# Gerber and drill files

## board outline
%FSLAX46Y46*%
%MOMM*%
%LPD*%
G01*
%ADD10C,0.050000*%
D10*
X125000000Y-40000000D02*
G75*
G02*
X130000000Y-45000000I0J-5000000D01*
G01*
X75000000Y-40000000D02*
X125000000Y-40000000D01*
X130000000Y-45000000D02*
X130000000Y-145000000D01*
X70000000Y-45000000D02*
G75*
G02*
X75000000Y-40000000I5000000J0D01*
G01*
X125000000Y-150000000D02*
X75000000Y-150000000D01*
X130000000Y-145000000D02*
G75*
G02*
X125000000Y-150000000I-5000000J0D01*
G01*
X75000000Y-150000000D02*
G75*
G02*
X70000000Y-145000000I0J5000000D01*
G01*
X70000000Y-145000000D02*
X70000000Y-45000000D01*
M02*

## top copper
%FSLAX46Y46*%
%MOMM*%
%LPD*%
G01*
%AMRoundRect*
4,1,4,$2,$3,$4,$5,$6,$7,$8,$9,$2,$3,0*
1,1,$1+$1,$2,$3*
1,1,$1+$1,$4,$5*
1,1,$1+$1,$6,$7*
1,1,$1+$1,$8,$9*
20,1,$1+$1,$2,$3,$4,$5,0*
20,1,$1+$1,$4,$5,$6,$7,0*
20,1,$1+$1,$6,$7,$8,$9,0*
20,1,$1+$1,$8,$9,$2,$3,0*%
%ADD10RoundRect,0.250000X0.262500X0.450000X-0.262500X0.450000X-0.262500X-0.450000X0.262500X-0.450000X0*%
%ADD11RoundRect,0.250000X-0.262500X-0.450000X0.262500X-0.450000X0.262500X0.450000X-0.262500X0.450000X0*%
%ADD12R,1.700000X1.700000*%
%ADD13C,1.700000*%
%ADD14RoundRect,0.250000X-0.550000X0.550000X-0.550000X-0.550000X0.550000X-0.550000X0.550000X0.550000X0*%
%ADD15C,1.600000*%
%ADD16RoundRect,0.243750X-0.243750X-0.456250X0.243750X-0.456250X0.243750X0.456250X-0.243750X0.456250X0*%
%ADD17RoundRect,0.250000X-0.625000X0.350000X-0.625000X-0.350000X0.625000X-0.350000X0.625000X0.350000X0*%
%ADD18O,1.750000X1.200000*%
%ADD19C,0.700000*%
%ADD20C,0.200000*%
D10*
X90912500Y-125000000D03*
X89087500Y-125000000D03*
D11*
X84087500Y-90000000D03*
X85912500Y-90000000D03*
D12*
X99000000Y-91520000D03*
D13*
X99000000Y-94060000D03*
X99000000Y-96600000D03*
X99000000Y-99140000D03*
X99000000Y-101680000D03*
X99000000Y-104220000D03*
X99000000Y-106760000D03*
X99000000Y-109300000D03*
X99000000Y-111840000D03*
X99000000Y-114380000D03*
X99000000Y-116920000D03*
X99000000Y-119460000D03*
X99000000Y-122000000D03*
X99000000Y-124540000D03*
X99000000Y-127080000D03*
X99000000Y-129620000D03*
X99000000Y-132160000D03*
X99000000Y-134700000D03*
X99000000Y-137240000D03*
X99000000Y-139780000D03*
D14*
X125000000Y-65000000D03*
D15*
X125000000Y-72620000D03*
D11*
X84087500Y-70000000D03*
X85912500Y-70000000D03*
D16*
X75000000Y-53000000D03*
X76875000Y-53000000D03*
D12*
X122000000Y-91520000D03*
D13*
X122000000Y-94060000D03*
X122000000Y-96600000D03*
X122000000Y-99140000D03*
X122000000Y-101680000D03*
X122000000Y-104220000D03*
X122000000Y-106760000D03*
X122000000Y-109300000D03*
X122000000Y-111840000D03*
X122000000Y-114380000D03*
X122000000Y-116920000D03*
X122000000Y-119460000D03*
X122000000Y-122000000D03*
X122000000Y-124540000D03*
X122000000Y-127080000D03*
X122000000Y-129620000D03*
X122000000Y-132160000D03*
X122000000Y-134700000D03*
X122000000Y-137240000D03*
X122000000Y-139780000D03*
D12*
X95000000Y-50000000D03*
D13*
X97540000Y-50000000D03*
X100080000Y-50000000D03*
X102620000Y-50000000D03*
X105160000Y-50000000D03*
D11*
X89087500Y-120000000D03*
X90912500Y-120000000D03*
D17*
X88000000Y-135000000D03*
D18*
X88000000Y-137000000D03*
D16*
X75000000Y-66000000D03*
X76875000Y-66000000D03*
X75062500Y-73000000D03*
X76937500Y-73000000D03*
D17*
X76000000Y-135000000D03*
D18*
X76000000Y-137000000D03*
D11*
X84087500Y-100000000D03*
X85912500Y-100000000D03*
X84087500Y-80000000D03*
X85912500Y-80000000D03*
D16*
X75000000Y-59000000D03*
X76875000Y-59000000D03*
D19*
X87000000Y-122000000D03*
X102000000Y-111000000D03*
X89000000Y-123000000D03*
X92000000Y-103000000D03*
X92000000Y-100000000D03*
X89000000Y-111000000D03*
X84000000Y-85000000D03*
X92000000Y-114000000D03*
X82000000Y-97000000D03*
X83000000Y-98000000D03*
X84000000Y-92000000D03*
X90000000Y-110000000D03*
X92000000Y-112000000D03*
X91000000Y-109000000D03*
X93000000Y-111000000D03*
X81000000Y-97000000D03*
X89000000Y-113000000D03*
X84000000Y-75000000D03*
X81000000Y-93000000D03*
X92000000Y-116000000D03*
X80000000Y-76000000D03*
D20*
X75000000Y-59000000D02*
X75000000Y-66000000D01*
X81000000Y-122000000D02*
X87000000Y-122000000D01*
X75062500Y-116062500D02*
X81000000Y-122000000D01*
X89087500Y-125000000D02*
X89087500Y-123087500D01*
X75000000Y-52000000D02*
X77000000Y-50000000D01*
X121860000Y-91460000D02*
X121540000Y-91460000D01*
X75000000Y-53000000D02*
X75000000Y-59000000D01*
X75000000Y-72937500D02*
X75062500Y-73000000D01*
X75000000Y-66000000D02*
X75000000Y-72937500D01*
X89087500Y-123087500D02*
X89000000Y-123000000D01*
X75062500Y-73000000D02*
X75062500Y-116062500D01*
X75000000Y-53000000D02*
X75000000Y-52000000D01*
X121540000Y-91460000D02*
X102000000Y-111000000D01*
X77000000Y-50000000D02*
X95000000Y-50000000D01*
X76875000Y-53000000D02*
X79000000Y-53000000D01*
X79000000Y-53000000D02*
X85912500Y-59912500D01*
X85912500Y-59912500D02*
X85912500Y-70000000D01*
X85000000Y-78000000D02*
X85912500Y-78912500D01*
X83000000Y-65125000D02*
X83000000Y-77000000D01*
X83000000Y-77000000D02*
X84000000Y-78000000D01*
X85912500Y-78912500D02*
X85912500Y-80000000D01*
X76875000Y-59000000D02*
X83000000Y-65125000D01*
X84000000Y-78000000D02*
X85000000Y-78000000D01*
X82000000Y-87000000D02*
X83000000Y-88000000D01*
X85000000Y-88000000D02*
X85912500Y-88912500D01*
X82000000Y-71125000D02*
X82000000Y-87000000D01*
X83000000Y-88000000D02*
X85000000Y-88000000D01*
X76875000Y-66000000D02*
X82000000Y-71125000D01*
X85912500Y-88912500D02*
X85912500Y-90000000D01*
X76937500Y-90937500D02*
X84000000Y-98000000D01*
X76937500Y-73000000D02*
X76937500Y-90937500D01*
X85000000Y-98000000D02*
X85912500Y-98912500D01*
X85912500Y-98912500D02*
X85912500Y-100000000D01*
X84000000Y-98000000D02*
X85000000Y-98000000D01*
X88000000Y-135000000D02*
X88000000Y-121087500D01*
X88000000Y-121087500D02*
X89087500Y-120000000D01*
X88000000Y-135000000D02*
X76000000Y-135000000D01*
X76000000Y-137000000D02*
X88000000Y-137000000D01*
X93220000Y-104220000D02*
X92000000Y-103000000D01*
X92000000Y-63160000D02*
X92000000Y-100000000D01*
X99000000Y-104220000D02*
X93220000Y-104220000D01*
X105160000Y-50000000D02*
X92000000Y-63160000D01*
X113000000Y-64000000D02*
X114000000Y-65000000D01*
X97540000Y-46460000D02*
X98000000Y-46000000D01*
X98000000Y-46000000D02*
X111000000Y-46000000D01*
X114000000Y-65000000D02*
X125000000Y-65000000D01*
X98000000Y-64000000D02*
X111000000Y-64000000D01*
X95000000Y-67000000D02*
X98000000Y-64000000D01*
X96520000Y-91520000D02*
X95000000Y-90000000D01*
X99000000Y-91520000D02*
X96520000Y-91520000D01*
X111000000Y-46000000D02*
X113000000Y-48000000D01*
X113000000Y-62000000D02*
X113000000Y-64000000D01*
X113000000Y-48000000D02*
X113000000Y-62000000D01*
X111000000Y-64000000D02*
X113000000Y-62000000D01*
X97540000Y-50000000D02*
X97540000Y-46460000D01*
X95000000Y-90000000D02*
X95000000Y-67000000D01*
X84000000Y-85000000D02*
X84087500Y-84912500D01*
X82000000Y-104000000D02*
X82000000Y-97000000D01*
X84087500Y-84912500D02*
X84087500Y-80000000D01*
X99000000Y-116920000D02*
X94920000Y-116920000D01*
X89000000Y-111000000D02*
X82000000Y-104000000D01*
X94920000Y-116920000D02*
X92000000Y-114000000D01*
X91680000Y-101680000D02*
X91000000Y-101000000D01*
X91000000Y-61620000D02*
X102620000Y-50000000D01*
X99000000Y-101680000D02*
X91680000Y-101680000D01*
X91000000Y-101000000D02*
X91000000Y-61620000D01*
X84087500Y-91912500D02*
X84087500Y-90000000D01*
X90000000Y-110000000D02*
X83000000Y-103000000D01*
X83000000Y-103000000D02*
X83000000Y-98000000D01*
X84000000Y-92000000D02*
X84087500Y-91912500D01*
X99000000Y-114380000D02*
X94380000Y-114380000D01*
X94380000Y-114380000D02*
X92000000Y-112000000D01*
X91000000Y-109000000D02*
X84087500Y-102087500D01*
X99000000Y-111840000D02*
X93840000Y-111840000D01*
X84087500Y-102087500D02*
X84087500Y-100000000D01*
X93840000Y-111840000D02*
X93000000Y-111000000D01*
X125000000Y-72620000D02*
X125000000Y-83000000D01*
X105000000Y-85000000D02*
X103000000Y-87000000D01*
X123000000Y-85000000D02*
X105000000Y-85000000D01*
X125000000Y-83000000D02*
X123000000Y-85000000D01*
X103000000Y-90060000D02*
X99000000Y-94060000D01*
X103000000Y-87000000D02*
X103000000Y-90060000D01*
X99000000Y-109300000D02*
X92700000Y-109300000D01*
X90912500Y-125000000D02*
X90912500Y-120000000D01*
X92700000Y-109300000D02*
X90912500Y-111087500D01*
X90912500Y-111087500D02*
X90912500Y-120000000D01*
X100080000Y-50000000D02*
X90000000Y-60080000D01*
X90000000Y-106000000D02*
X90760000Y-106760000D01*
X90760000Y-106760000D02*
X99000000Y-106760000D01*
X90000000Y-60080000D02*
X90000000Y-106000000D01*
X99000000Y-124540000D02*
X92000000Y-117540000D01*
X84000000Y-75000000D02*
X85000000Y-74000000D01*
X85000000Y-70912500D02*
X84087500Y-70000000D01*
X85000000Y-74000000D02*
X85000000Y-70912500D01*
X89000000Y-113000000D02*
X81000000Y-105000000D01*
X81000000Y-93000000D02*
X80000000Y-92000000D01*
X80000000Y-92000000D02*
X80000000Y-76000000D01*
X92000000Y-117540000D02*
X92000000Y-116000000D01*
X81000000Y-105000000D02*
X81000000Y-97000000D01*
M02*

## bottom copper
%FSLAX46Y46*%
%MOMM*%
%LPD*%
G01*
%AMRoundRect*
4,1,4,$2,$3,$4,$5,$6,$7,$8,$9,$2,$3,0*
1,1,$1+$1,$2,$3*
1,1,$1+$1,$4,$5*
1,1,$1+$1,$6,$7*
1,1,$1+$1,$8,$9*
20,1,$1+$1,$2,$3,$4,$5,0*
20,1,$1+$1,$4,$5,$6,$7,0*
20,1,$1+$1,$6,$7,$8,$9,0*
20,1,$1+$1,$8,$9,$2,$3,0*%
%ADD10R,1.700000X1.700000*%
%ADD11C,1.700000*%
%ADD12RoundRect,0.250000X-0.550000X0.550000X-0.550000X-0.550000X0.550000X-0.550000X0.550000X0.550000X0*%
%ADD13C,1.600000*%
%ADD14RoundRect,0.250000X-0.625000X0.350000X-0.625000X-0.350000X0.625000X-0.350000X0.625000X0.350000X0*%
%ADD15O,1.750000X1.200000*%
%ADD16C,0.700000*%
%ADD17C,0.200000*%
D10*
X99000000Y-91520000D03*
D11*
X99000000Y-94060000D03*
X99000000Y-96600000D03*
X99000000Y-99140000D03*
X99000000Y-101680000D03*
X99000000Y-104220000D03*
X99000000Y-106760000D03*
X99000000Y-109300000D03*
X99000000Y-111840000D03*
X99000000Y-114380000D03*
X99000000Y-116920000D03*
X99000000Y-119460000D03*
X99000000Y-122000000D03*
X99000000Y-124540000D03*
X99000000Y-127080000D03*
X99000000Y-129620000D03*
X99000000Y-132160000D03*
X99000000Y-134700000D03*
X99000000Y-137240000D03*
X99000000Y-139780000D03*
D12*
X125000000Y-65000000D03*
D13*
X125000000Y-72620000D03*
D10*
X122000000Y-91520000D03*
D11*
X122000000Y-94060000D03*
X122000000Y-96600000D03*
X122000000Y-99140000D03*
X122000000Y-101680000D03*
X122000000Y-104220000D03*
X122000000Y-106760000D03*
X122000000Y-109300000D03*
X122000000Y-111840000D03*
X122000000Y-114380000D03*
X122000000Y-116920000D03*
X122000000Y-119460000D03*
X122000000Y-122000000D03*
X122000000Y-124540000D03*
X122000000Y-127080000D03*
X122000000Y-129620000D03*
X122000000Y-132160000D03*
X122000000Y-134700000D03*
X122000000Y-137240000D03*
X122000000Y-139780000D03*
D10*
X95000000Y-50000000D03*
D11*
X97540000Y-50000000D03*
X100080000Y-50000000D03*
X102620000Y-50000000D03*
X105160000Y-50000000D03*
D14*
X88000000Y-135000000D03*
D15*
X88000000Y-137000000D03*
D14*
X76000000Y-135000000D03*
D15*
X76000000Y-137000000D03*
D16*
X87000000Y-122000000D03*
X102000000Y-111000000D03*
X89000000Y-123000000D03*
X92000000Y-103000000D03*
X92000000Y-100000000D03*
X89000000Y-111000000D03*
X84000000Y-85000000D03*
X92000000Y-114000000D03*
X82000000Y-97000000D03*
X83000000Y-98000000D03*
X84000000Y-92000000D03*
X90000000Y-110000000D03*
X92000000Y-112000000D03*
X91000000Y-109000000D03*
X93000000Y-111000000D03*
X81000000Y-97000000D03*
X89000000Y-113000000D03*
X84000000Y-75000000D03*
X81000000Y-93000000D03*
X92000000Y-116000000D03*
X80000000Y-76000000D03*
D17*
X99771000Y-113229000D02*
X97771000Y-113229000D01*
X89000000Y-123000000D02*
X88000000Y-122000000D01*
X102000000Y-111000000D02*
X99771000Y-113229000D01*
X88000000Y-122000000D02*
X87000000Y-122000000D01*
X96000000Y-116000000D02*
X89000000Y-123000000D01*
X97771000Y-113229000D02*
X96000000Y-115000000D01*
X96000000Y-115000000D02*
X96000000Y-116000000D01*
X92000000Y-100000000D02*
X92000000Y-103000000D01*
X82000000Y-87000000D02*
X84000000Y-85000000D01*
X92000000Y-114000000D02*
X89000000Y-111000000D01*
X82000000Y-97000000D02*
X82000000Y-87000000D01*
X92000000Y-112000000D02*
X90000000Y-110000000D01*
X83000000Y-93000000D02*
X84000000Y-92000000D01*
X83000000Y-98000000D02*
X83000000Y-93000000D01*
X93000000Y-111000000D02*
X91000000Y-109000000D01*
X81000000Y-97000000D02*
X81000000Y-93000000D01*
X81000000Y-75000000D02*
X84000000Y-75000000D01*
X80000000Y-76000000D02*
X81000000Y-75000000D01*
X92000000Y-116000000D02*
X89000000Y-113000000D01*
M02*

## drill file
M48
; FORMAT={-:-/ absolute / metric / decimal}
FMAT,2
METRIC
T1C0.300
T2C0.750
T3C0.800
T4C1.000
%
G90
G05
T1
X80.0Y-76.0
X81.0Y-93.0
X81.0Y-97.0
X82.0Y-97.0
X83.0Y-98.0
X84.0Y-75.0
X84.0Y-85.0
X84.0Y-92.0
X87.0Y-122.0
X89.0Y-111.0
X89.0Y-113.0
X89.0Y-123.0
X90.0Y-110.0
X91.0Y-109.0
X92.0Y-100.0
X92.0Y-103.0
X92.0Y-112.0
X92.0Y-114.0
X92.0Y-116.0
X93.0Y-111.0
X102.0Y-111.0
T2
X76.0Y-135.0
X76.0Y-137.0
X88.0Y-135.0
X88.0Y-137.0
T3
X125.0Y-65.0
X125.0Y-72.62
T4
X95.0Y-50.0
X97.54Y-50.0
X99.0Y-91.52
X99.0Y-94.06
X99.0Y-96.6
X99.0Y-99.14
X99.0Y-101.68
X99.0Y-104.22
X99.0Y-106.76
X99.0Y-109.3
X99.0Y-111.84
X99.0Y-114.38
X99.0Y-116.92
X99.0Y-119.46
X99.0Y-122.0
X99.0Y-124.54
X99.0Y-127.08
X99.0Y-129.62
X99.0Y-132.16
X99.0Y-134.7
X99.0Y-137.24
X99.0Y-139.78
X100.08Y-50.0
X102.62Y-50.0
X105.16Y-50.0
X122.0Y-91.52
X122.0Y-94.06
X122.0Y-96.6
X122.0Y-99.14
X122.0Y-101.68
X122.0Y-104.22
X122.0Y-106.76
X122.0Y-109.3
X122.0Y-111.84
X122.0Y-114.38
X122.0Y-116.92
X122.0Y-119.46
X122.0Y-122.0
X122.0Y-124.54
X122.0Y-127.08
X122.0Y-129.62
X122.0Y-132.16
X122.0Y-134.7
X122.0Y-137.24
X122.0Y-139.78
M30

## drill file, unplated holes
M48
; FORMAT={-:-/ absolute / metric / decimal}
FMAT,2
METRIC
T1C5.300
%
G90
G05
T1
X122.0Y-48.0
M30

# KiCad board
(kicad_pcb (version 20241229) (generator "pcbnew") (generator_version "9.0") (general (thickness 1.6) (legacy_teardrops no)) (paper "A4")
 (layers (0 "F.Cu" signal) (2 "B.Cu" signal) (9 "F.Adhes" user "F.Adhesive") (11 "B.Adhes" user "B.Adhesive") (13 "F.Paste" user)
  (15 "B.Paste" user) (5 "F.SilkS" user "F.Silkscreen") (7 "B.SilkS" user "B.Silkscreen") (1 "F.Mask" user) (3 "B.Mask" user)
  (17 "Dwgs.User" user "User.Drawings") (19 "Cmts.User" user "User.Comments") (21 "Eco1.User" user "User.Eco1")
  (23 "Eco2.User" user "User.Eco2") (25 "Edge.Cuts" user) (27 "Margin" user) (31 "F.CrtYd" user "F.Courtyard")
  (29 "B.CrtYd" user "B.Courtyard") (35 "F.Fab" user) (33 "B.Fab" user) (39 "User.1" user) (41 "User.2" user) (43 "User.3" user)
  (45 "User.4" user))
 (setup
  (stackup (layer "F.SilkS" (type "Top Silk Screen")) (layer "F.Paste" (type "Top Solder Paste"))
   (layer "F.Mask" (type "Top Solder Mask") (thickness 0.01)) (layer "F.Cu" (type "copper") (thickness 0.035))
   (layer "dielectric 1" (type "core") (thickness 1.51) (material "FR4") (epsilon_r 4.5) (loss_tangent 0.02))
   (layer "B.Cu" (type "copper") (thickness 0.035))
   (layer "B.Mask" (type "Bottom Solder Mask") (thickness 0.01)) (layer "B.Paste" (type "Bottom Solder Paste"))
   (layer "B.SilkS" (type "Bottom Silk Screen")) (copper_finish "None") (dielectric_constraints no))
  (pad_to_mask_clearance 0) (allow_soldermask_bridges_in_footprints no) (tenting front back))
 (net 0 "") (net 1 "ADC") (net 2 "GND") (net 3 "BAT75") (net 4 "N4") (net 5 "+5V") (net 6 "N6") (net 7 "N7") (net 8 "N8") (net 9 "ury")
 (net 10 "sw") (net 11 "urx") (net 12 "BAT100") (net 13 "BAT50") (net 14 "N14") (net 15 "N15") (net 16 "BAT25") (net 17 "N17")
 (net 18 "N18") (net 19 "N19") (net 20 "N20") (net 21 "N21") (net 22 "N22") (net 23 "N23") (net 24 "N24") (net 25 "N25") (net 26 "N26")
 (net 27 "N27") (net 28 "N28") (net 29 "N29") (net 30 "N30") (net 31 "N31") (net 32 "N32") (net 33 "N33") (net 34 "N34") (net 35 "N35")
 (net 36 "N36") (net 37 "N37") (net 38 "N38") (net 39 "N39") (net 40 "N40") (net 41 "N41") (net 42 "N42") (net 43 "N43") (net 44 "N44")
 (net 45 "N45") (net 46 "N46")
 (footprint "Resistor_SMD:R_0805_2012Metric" (layer "F.Cu") (at 90 125 180)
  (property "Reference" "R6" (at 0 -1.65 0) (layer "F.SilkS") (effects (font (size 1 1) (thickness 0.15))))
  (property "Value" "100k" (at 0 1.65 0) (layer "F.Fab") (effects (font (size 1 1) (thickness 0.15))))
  (pad "1" smd roundrect (at -0.9125 0 180) (size 1.025 1.4) (layers "F.Cu" "F.Mask" "F.Paste") (roundrect_rratio 0.243902) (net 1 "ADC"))
  (pad "2" smd roundrect (at 0.9125 0 180) (size 1.025 1.4) (layers "F.Cu" "F.Mask" "F.Paste") (roundrect_rratio 0.243902) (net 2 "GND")))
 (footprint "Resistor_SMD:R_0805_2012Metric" (layer "F.Cu") (at 85 90)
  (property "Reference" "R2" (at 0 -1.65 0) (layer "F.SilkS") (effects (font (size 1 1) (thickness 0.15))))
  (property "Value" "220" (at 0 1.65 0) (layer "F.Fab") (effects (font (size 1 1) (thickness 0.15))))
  (pad "1" smd roundrect (at -0.9125 0) (size 1.025 1.4) (layers "F.Cu" "F.Mask" "F.Paste") (roundrect_rratio 0.243902) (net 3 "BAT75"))
  (pad "2" smd roundrect (at 0.9125 0) (size 1.025 1.4) (layers "F.Cu" "F.Mask" "F.Paste") (roundrect_rratio 0.243902) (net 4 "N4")))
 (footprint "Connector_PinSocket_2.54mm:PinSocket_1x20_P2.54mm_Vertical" (layer "F.Cu") (at 99 91.52)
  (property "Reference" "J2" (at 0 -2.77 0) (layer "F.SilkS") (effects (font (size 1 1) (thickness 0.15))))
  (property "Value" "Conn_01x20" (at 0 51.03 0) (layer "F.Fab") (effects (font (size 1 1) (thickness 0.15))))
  (pad "1" thru_hole rect (at 0 0) (size 1.7 1.7) (drill 1) (layers "*.Cu" "*.Mask") (remove_unused_layers no) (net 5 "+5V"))
  (pad "2" thru_hole circle (at 0 2.54) (size 1.7 1.7) (drill 1) (layers "*.Cu" "*.Mask") (remove_unused_layers no) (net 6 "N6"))
  (pad "3" thru_hole circle (at 0 5.08) (size 1.7 1.7) (drill 1) (layers "*.Cu" "*.Mask") (remove_unused_layers no) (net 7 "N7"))
  (pad "4" thru_hole circle (at 0 7.62) (size 1.7 1.7) (drill 1) (layers "*.Cu" "*.Mask") (remove_unused_layers no) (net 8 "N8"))
  (pad "5" thru_hole circle (at 0 10.16) (size 1.7 1.7) (drill 1) (layers "*.Cu" "*.Mask") (remove_unused_layers no) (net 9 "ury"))
  (pad "6" thru_hole circle (at 0 12.7) (size 1.7 1.7) (drill 1) (layers "*.Cu" "*.Mask") (remove_unused_layers no) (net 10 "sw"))
  (pad "7" thru_hole circle (at 0 15.24) (size 1.7 1.7) (drill 1) (layers "*.Cu" "*.Mask") (remove_unused_layers no) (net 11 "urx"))
  (pad "8" thru_hole circle (at 0 17.78) (size 1.7 1.7) (drill 1) (layers "*.Cu" "*.Mask") (remove_unused_layers no) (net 1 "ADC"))
  (pad "9" thru_hole circle (at 0 20.32) (size 1.7 1.7) (drill 1) (layers "*.Cu" "*.Mask") (remove_unused_layers no) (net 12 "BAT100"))
  (pad "10" thru_hole circle (at 0 22.86) (size 1.7 1.7) (drill 1) (layers "*.Cu" "*.Mask") (remove_unused_layers no) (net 3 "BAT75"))
  (pad "11" thru_hole circle (at 0 25.4) (size 1.7 1.7) (drill 1) (layers "*.Cu" "*.Mask") (remove_unused_layers no) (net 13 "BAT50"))
  (pad "12" thru_hole circle (at 0 27.94) (size 1.7 1.7) (drill 1) (layers "*.Cu" "*.Mask") (remove_unused_layers no) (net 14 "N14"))
  (pad "13" thru_hole circle (at 0 30.48) (size 1.7 1.7) (drill 1) (layers "*.Cu" "*.Mask") (remove_unused_layers no) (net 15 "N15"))
  (pad "14" thru_hole circle (at 0 33.02) (size 1.7 1.7) (drill 1) (layers "*.Cu" "*.Mask") (remove_unused_layers no) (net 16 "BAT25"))
  (pad "15" thru_hole circle (at 0 35.56) (size 1.7 1.7) (drill 1) (layers "*.Cu" "*.Mask") (remove_unused_layers no) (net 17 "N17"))
  (pad "16" thru_hole circle (at 0 38.1) (size 1.7 1.7) (drill 1) (layers "*.Cu" "*.Mask") (remove_unused_layers no) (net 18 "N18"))
  (pad "17" thru_hole circle (at 0 40.64) (size 1.7 1.7) (drill 1) (layers "*.Cu" "*.Mask") (remove_unused_layers no) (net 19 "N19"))
  (pad "18" thru_hole circle (at 0 43.18) (size 1.7 1.7) (drill 1) (layers "*.Cu" "*.Mask") (remove_unused_layers no) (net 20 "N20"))
  (pad "19" thru_hole circle (at 0 45.72) (size 1.7 1.7) (drill 1) (layers "*.Cu" "*.Mask") (remove_unused_layers no) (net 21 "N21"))
  (pad "20" thru_hole circle (at 0 48.26) (size 1.7 1.7) (drill 1) (layers "*.Cu" "*.Mask") (remove_unused_layers no) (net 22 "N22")))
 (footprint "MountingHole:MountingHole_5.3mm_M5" (layer "F.Cu") (at 122 48)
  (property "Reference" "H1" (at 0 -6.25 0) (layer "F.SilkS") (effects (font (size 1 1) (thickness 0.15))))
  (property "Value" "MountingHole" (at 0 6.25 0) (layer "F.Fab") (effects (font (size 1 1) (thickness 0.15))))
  (pad "" np_thru_hole circle (at 0 0) (size 5.3 5.3) (drill 5.3) (layers "*.Cu" "*.Mask")))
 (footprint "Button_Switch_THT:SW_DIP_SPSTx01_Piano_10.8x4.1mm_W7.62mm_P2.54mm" (layer "F.Cu") (at 125 65 -90)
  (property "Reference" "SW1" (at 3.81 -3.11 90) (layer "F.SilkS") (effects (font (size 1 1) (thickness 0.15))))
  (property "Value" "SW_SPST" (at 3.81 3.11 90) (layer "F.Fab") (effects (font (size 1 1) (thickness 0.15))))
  (pad "1" thru_hole roundrect (at 0 0 270) (size 1.6 1.6) (drill 0.8) (layers "*.Cu" "*.Mask") (remove_unused_layers no)
   (roundrect_rratio 0.15625) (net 5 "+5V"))
  (pad "2" thru_hole circle (at 7.62 0 270) (size 1.6 1.6) (drill 0.8) (layers "*.Cu" "*.Mask") (remove_unused_layers no) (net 6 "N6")))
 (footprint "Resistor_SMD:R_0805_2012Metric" (layer "F.Cu") (at 85 70)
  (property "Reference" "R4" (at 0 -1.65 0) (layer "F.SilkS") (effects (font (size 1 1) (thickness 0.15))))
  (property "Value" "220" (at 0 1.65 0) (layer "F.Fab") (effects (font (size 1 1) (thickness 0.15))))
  (pad "1" smd roundrect (at -0.9125 0) (size 1.025 1.4) (layers "F.Cu" "F.Mask" "F.Paste") (roundrect_rratio 0.243902) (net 16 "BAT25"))
  (pad "2" smd roundrect (at 0.9125 0) (size 1.025 1.4) (layers "F.Cu" "F.Mask" "F.Paste") (roundrect_rratio 0.243902) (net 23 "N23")))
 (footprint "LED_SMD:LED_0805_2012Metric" (layer "F.Cu") (at 75.9375 53)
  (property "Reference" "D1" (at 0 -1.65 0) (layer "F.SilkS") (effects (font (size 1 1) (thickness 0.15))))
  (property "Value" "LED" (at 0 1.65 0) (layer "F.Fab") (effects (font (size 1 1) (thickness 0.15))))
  (pad "1" smd roundrect (at -0.9375 0) (size 0.975 1.4) (layers "F.Cu" "F.Mask" "F.Paste") (roundrect_rratio 0.25) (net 2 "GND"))
  (pad "2" smd roundrect (at 0.9375 0) (size 0.975 1.4) (layers "F.Cu" "F.Mask" "F.Paste") (roundrect_rratio 0.25) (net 23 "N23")))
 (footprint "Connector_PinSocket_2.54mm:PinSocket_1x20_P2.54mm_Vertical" (layer "F.Cu") (at 122 91.52)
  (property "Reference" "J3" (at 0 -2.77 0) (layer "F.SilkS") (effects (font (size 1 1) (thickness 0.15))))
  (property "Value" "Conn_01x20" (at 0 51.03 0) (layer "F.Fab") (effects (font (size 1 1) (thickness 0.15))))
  (pad "1" thru_hole rect (at 0 0) (size 1.7 1.7) (drill 1) (layers "*.Cu" "*.Mask") (remove_unused_layers no) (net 2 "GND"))
  (pad "2" thru_hole circle (at 0 2.54) (size 1.7 1.7) (drill 1) (layers "*.Cu" "*.Mask") (remove_unused_layers no) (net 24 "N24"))
  (pad "3" thru_hole circle (at 0 5.08) (size 1.7 1.7) (drill 1) (layers "*.Cu" "*.Mask") (remove_unused_layers no) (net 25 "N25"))
  (pad "4" thru_hole circle (at 0 7.62) (size 1.7 1.7) (drill 1) (layers "*.Cu" "*.Mask") (remove_unused_layers no) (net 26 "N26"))
  (pad "5" thru_hole circle (at 0 10.16) (size 1.7 1.7) (drill 1) (layers "*.Cu" "*.Mask") (remove_unused_layers no) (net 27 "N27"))
  (pad "6" thru_hole circle (at 0 12.7) (size 1.7 1.7) (drill 1) (layers "*.Cu" "*.Mask") (remove_unused_layers no) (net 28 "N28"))
  (pad "7" thru_hole circle (at 0 15.24) (size 1.7 1.7) (drill 1) (layers "*.Cu" "*.Mask") (remove_unused_layers no) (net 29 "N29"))
  (pad "8" thru_hole circle (at 0 17.78) (size 1.7 1.7) (drill 1) (layers "*.Cu" "*.Mask") (remove_unused_layers no) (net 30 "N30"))
  (pad "9" thru_hole circle (at 0 20.32) (size 1.7 1.7) (drill 1) (layers "*.Cu" "*.Mask") (remove_unused_layers no) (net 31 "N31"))
  (pad "10" thru_hole circle (at 0 22.86) (size 1.7 1.7) (drill 1) (layers "*.Cu" "*.Mask") (remove_unused_layers no) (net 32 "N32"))
  (pad "11" thru_hole circle (at 0 25.4) (size 1.7 1.7) (drill 1) (layers "*.Cu" "*.Mask") (remove_unused_layers no) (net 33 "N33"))
  (pad "12" thru_hole circle (at 0 27.94) (size 1.7 1.7) (drill 1) (layers "*.Cu" "*.Mask") (remove_unused_layers no) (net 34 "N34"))
  (pad "13" thru_hole circle (at 0 30.48) (size 1.7 1.7) (drill 1) (layers "*.Cu" "*.Mask") (remove_unused_layers no) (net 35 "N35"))
  (pad "14" thru_hole circle (at 0 33.02) (size 1.7 1.7) (drill 1) (layers "*.Cu" "*.Mask") (remove_unused_layers no) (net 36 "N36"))
  (pad "15" thru_hole circle (at 0 35.56) (size 1.7 1.7) (drill 1) (layers "*.Cu" "*.Mask") (remove_unused_layers no) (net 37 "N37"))
  (pad "16" thru_hole circle (at 0 38.1) (size 1.7 1.7) (drill 1) (layers "*.Cu" "*.Mask") (remove_unused_layers no) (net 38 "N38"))
  (pad "17" thru_hole circle (at 0 40.64) (size 1.7 1.7) (drill 1) (layers "*.Cu" "*.Mask") (remove_unused_layers no) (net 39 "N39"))
  (pad "18" thru_hole circle (at 0 43.18) (size 1.7 1.7) (drill 1) (layers "*.Cu" "*.Mask") (remove_unused_layers no) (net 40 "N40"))
  (pad "19" thru_hole circle (at 0 45.72) (size 1.7 1.7) (drill 1) (layers "*.Cu" "*.Mask") (remove_unused_layers no) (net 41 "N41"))
  (pad "20" thru_hole circle (at 0 48.26) (size 1.7 1.7) (drill 1) (layers "*.Cu" "*.Mask") (remove_unused_layers no) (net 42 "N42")))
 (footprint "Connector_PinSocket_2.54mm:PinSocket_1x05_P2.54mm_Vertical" (layer "F.Cu") (at 95 50 90)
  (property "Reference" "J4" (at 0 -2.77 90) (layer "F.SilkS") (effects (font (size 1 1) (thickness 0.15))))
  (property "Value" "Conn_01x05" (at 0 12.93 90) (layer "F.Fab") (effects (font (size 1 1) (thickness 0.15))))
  (pad "1" thru_hole rect (at 0 0 90) (size 1.7 1.7) (drill 1) (layers "*.Cu" "*.Mask") (remove_unused_layers no) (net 2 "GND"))
  (pad "2" thru_hole circle (at 0 2.54 90) (size 1.7 1.7) (drill 1) (layers "*.Cu" "*.Mask") (remove_unused_layers no) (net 5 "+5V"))
  (pad "3" thru_hole circle (at 0 5.08 90) (size 1.7 1.7) (drill 1) (layers "*.Cu" "*.Mask") (remove_unused_layers no) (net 11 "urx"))
  (pad "4" thru_hole circle (at 0 7.62 90) (size 1.7 1.7) (drill 1) (layers "*.Cu" "*.Mask") (remove_unused_layers no) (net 9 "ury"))
  (pad "5" thru_hole circle (at 0 10.16 90) (size 1.7 1.7) (drill 1) (layers "*.Cu" "*.Mask") (remove_unused_layers no) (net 10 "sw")))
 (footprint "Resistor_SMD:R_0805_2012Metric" (layer "F.Cu") (at 90 120)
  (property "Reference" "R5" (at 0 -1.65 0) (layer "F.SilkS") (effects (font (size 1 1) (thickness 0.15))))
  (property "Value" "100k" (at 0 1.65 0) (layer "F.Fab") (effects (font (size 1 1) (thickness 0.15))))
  (pad "1" smd roundrect (at -0.9125 0) (size 1.025 1.4) (layers "F.Cu" "F.Mask" "F.Paste") (roundrect_rratio 0.243902) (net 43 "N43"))
  (pad "2" smd roundrect (at 0.9125 0) (size 1.025 1.4) (layers "F.Cu" "F.Mask" "F.Paste") (roundrect_rratio 0.243902) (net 1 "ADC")))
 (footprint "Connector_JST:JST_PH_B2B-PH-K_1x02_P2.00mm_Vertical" (layer "F.Cu") (at 88 135 -90)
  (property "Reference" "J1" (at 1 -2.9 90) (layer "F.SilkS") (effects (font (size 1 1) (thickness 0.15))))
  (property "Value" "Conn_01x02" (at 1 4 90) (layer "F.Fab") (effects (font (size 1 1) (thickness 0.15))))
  (pad "1" thru_hole roundrect (at 0 0 270) (size 1.2 1.75) (drill 0.75) (layers "*.Cu" "*.Mask") (remove_unused_layers no)
   (roundrect_rratio 0.208333) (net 43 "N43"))
  (pad "2" thru_hole oval (at 2 0 270) (size 1.2 1.75) (drill 0.75) (layers "*.Cu" "*.Mask") (remove_unused_layers no) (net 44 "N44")))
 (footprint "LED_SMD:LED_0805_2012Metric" (layer "F.Cu") (at 75.9375 66)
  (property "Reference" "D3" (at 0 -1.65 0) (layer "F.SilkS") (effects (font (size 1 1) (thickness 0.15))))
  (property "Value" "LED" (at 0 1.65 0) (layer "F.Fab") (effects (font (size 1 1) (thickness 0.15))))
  (pad "1" smd roundrect (at -0.9375 0) (size 0.975 1.4) (layers "F.Cu" "F.Mask" "F.Paste") (roundrect_rratio 0.25) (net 2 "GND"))
  (pad "2" smd roundrect (at 0.9375 0) (size 0.975 1.4) (layers "F.Cu" "F.Mask" "F.Paste") (roundrect_rratio 0.25) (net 4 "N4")))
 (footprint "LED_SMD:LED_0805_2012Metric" (layer "F.Cu") (at 76 73)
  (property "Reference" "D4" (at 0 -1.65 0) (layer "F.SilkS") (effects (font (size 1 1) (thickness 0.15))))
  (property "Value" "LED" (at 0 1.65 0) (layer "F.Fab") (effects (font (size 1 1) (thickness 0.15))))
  (pad "1" smd roundrect (at -0.9375 0) (size 0.975 1.4) (layers "F.Cu" "F.Mask" "F.Paste") (roundrect_rratio 0.25) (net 2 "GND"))
  (pad "2" smd roundrect (at 0.9375 0) (size 0.975 1.4) (layers "F.Cu" "F.Mask" "F.Paste") (roundrect_rratio 0.25) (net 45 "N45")))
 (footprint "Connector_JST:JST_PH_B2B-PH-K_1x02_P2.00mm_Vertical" (layer "F.Cu") (at 76 135 -90)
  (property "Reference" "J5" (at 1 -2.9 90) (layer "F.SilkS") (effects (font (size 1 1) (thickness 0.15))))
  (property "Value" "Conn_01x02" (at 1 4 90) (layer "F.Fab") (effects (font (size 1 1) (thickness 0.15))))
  (pad "1" thru_hole roundrect (at 0 0 270) (size 1.2 1.75) (drill 0.75) (layers "*.Cu" "*.Mask") (remove_unused_layers no)
   (roundrect_rratio 0.208333) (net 43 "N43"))
  (pad "2" thru_hole oval (at 2 0 270) (size 1.2 1.75) (drill 0.75) (layers "*.Cu" "*.Mask") (remove_unused_layers no) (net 44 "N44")))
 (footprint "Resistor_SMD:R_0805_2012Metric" (layer "F.Cu") (at 85 100)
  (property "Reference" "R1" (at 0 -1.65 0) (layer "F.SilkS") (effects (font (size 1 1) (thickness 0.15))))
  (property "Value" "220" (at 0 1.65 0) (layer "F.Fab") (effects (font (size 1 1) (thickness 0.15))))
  (pad "1" smd roundrect (at -0.9125 0) (size 1.025 1.4) (layers "F.Cu" "F.Mask" "F.Paste") (roundrect_rratio 0.243902) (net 12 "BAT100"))
  (pad "2" smd roundrect (at 0.9125 0) (size 1.025 1.4) (layers "F.Cu" "F.Mask" "F.Paste") (roundrect_rratio 0.243902) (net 45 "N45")))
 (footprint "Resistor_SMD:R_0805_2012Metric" (layer "F.Cu") (at 85 80)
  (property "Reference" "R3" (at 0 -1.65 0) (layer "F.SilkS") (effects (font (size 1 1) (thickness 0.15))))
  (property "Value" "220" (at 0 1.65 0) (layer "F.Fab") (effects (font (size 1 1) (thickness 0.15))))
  (pad "1" smd roundrect (at -0.9125 0) (size 1.025 1.4) (layers "F.Cu" "F.Mask" "F.Paste") (roundrect_rratio 0.243902) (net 13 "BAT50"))
  (pad "2" smd roundrect (at 0.9125 0) (size 1.025 1.4) (layers "F.Cu" "F.Mask" "F.Paste") (roundrect_rratio 0.243902) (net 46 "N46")))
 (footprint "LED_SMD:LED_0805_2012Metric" (layer "F.Cu") (at 75.9375 59)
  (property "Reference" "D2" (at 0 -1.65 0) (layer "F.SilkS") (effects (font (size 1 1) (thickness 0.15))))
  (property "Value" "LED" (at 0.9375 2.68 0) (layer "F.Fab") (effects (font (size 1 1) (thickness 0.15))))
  (pad "1" smd roundrect (at -0.9375 0) (size 0.975 1.4) (layers "F.Cu" "F.Mask" "F.Paste") (roundrect_rratio 0.25) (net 2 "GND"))
  (pad "2" smd roundrect (at 0.9375 0) (size 0.975 1.4) (layers "F.Cu" "F.Mask" "F.Paste") (roundrect_rratio 0.25) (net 46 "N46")))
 (gr_arc (start 125 40) (mid 128.535534 41.464466) (end 130 45) (stroke (width 0.05) (type default)) (layer "Edge.Cuts"))
 (gr_line (start 75 40) (end 125 40) (stroke (width 0.05) (type default)) (layer "Edge.Cuts"))
 (gr_line (start 130 45) (end 130 145) (stroke (width 0.05) (type default)) (layer "Edge.Cuts"))
 (gr_arc (start 70 45) (mid 71.464466 41.464466) (end 75 40) (stroke (width 0.05) (type default)) (layer "Edge.Cuts"))
 (gr_line (start 125 150) (end 75 150) (stroke (width 0.05) (type default)) (layer "Edge.Cuts"))
 (gr_arc (start 130 145) (mid 128.535534 148.535534) (end 125 150) (stroke (width 0.05) (type default)) (layer "Edge.Cuts"))
 (gr_line (start 70 145) (end 70 45) (stroke (width 0.05) (type default)) (layer "Edge.Cuts"))
 (gr_arc (start 75 150) (mid 71.464466 148.535534) (end 70 145) (stroke (width 0.05) (type default)) (layer "Edge.Cuts"))
 (segment (start 75 59) (end 75 66) (width 0.2) (layer "F.Cu") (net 2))
 (segment (start 81 122) (end 87 122) (width 0.2) (layer "F.Cu") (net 2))
 (segment (start 75.0625 116.0625) (end 81 122) (width 0.2) (layer "F.Cu") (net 2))
 (segment (start 89.0875 125) (end 89.0875 123.0875) (width 0.2) (layer "F.Cu") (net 2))
 (segment (start 75 52) (end 77 50) (width 0.2) (layer "F.Cu") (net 2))
 (segment (start 121.86 91.46) (end 121.54 91.46) (width 0.2) (layer "F.Cu") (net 2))
 (segment (start 75 53) (end 75 59) (width 0.2) (layer "F.Cu") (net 2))
 (segment (start 75 72.9375) (end 75.0625 73) (width 0.2) (layer "F.Cu") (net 2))
 (segment (start 75 66) (end 75 72.9375) (width 0.2) (layer "F.Cu") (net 2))
 (segment (start 89.0875 123.0875) (end 89 123) (width 0.2) (layer "F.Cu") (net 2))
 (segment (start 75.0625 73) (end 75.0625 116.0625) (width 0.2) (layer "F.Cu") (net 2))
 (segment (start 75 53) (end 75 52) (width 0.2) (layer "F.Cu") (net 2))
 (segment (start 121.54 91.46) (end 102 111) (width 0.2) (layer "F.Cu") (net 2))
 (segment (start 77 50) (end 95 50) (width 0.2) (layer "F.Cu") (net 2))
 (via (at 87 122) (size 0.7) (drill 0.3) (layers "F.Cu" "B.Cu") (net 2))
 (via (at 102 111) (size 0.7) (drill 0.3) (layers "F.Cu" "B.Cu") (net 2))
 (via (at 89 123) (size 0.7) (drill 0.3) (layers "F.Cu" "B.Cu") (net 2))
 (segment (start 99.771 113.229) (end 97.771 113.229) (width 0.2) (layer "B.Cu") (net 2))
 (segment (start 89 123) (end 88 122) (width 0.2) (layer "B.Cu") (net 2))
 (segment (start 102 111) (end 99.771 113.229) (width 0.2) (layer "B.Cu") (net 2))
 (segment (start 88 122) (end 87 122) (width 0.2) (layer "B.Cu") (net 2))
 (segment (start 96 116) (end 89 123) (width 0.2) (layer "B.Cu") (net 2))
 (segment (start 97.771 113.229) (end 96 115) (width 0.2) (layer "B.Cu") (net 2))
 (segment (start 96 115) (end 96 116) (width 0.2) (layer "B.Cu") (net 2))
 (segment (start 76.875 53) (end 79 53) (width 0.2) (layer "F.Cu") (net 23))
 (segment (start 79 53) (end 85.9125 59.9125) (width 0.2) (layer "F.Cu") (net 23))
 (segment (start 85.9125 59.9125) (end 85.9125 70) (width 0.2) (layer "F.Cu") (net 23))
 (segment (start 85 78) (end 85.9125 78.9125) (width 0.2) (layer "F.Cu") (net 46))
 (segment (start 83 65.125) (end 83 77) (width 0.2) (layer "F.Cu") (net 46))
 (segment (start 83 77) (end 84 78) (width 0.2) (layer "F.Cu") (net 46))
 (segment (start 85.9125 78.9125) (end 85.9125 80) (width 0.2) (layer "F.Cu") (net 46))
 (segment (start 76.875 59) (end 83 65.125) (width 0.2) (layer "F.Cu") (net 46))
 (segment (start 84 78) (end 85 78) (width 0.2) (layer "F.Cu") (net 46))
 (segment (start 82 87) (end 83 88) (width 0.2) (layer "F.Cu") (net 4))
 (segment (start 85 88) (end 85.9125 88.9125) (width 0.2) (layer "F.Cu") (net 4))
 (segment (start 82 71.125) (end 82 87) (width 0.2) (layer "F.Cu") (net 4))
 (segment (start 83 88) (end 85 88) (width 0.2) (layer "F.Cu") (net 4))
 (segment (start 76.875 66) (end 82 71.125) (width 0.2) (layer "F.Cu") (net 4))
 (segment (start 85.9125 88.9125) (end 85.9125 90) (width 0.2) (layer "F.Cu") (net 4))
 (segment (start 76.9375 90.9375) (end 84 98) (width 0.2) (layer "F.Cu") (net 45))
 (segment (start 76.9375 73) (end 76.9375 90.9375) (width 0.2) (layer "F.Cu") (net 45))
 (segment (start 85 98) (end 85.9125 98.9125) (width 0.2) (layer "F.Cu") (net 45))
 (segment (start 85.9125 98.9125) (end 85.9125 100) (width 0.2) (layer "F.Cu") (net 45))
 (segment (start 84 98) (end 85 98) (width 0.2) (layer "F.Cu") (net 45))
 (segment (start 88 135) (end 88 121.0875) (width 0.2) (layer "F.Cu") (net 43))
 (segment (start 88 121.0875) (end 89.0875 120) (width 0.2) (layer "F.Cu") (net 43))
 (segment (start 88 135) (end 76 135) (width 0.2) (layer "F.Cu") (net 43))
 (segment (start 76 137) (end 88 137) (width 0.2) (layer "F.Cu") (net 44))
 (segment (start 93.22 104.22) (end 92 103) (width 0.2) (layer "F.Cu") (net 10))
 (segment (start 92 63.16) (end 92 100) (width 0.2) (layer "F.Cu") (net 10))
 (segment (start 99 104.22) (end 93.22 104.22) (width 0.2) (layer "F.Cu") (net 10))
 (segment (start 105.16 50) (end 92 63.16) (width 0.2) (layer "F.Cu") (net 10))
 (via (at 92 103) (size 0.7) (drill 0.3) (layers "F.Cu" "B.Cu") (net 10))
 (via (at 92 100) (size 0.7) (drill 0.3) (layers "F.Cu" "B.Cu") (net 10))
 (segment (start 92 100) (end 92 103) (width 0.2) (layer "B.Cu") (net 10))
 (segment (start 113 64) (end 114 65) (width 0.2) (layer "F.Cu") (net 5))
 (segment (start 97.54 46.46) (end 98 46) (width 0.2) (layer "F.Cu") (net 5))
 (segment (start 98 46) (end 111 46) (width 0.2) (layer "F.Cu") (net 5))
 (segment (start 114 65) (end 125 65) (width 0.2) (layer "F.Cu") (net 5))
 (segment (start 98 64) (end 111 64) (width 0.2) (layer "F.Cu") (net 5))
 (segment (start 95 67) (end 98 64) (width 0.2) (layer "F.Cu") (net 5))
 (segment (start 96.52 91.52) (end 95 90) (width 0.2) (layer "F.Cu") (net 5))
 (segment (start 99 91.52) (end 96.52 91.52) (width 0.2) (layer "F.Cu") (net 5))
 (segment (start 111 46) (end 113 48) (width 0.2) (layer "F.Cu") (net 5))
 (segment (start 113 62) (end 113 64) (width 0.2) (layer "F.Cu") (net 5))
 (segment (start 113 48) (end 113 62) (width 0.2) (layer "F.Cu") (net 5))
 (segment (start 111 64) (end 113 62) (width 0.2) (layer "F.Cu") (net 5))
 (segment (start 97.54 50) (end 97.54 46.46) (width 0.2) (layer "F.Cu") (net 5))
 (segment (start 95 90) (end 95 67) (width 0.2) (layer "F.Cu") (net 5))
 (segment (start 84 85) (end 84.0875 84.9125) (width 0.2) (layer "F.Cu") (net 13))
 (segment (start 82 104) (end 82 97) (width 0.2) (layer "F.Cu") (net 13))
 (segment (start 84.0875 84.9125) (end 84.0875 80) (width 0.2) (layer "F.Cu") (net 13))
 (segment (start 99 116.92) (end 94.92 116.92) (width 0.2) (layer "F.Cu") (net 13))
 (segment (start 89 111) (end 82 104) (width 0.2) (layer "F.Cu") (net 13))
 (segment (start 94.92 116.92) (end 92 114) (width 0.2) (layer "F.Cu") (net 13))
 (via (at 89 111) (size 0.7) (drill 0.3) (layers "F.Cu" "B.Cu") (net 13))
 (via (at 84 85) (size 0.7) (drill 0.3) (layers "F.Cu" "B.Cu") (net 13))
 (via (at 92 114) (size 0.7) (drill 0.3) (layers "F.Cu" "B.Cu") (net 13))
 (via (at 82 97) (size 0.7) (drill 0.3) (layers "F.Cu" "B.Cu") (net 13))
 (segment (start 82 87) (end 84 85) (width 0.2) (layer "B.Cu") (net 13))
 (segment (start 92 114) (end 89 111) (width 0.2) (layer "B.Cu") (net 13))
 (segment (start 82 97) (end 82 87) (width 0.2) (layer "B.Cu") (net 13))
 (segment (start 91.68 101.68) (end 91 101) (width 0.2) (layer "F.Cu") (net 9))
 (segment (start 91 61.62) (end 102.62 50) (width 0.2) (layer "F.Cu") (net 9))
 (segment (start 99 101.68) (end 91.68 101.68) (width 0.2) (layer "F.Cu") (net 9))
 (segment (start 91 101) (end 91 61.62) (width 0.2) (layer "F.Cu") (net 9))
 (segment (start 84.0875 91.9125) (end 84.0875 90) (width 0.2) (layer "F.Cu") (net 3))
 (segment (start 90 110) (end 83 103) (width 0.2) (layer "F.Cu") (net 3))
 (segment (start 83 103) (end 83 98) (width 0.2) (layer "F.Cu") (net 3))
 (segment (start 84 92) (end 84.0875 91.9125) (width 0.2) (layer "F.Cu") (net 3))
 (segment (start 99 114.38) (end 94.38 114.38) (width 0.2) (layer "F.Cu") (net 3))
 (segment (start 94.38 114.38) (end 92 112) (width 0.2) (layer "F.Cu") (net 3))
 (via (at 83 98) (size 0.7) (drill 0.3) (layers "F.Cu" "B.Cu") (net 3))
 (via (at 84 92) (size 0.7) (drill 0.3) (layers "F.Cu" "B.Cu") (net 3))
 (via (at 90 110) (size 0.7) (drill 0.3) (layers "F.Cu" "B.Cu") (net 3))
 (via (at 92 112) (size 0.7) (drill 0.3) (layers "F.Cu" "B.Cu") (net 3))
 (segment (start 92 112) (end 90 110) (width 0.2) (layer "B.Cu") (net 3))
 (segment (start 83 93) (end 84 92) (width 0.2) (layer "B.Cu") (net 3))
 (segment (start 83 98) (end 83 93) (width 0.2) (layer "B.Cu") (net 3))
 (segment (start 91 109) (end 84.0875 102.0875) (width 0.2) (layer "F.Cu") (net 12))
 (segment (start 99 111.84) (end 93.84 111.84) (width 0.2) (layer "F.Cu") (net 12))
 (segment (start 84.0875 102.0875) (end 84.0875 100) (width 0.2) (layer "F.Cu") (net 12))
 (segment (start 93.84 111.84) (end 93 111) (width 0.2) (layer "F.Cu") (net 12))
 (via (at 91 109) (size 0.7) (drill 0.3) (layers "F.Cu" "B.Cu") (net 12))
 (via (at 93 111) (size 0.7) (drill 0.3) (layers "F.Cu" "B.Cu") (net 12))
 (segment (start 93 111) (end 91 109) (width 0.2) (layer "B.Cu") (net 12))
 (segment (start 125 72.62) (end 125 83) (width 0.2) (layer "F.Cu") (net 6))
 (segment (start 105 85) (end 103 87) (width 0.2) (layer "F.Cu") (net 6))
 (segment (start 123 85) (end 105 85) (width 0.2) (layer "F.Cu") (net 6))
 (segment (start 125 83) (end 123 85) (width 0.2) (layer "F.Cu") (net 6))
 (segment (start 103 90.06) (end 99 94.06) (width 0.2) (layer "F.Cu") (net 6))
 (segment (start 103 87) (end 103 90.06) (width 0.2) (layer "F.Cu") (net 6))
 (segment (start 99 109.3) (end 92.7 109.3) (width 0.2) (layer "F.Cu") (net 1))
 (segment (start 90.9125 125) (end 90.9125 120) (width 0.2) (layer "F.Cu") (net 1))
 (segment (start 92.7 109.3) (end 90.9125 111.0875) (width 0.2) (layer "F.Cu") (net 1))
 (segment (start 90.9125 111.0875) (end 90.9125 120) (width 0.2) (layer "F.Cu") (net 1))
 (segment (start 100.08 50) (end 90 60.08) (width 0.2) (layer "F.Cu") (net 11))
 (segment (start 90 106) (end 90.76 106.76) (width 0.2) (layer "F.Cu") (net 11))
 (segment (start 90.76 106.76) (end 99 106.76) (width 0.2) (layer "F.Cu") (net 11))
 (segment (start 90 60.08) (end 90 106) (width 0.2) (layer "F.Cu") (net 11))
 (segment (start 99 124.54) (end 92 117.54) (width 0.2) (layer "F.Cu") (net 16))
 (segment (start 84 75) (end 85 74) (width 0.2) (layer "F.Cu") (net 16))
 (segment (start 85 70.9125) (end 84.0875 70) (width 0.2) (layer "F.Cu") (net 16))
 (segment (start 85 74) (end 85 70.9125) (width 0.2) (layer "F.Cu") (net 16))
 (segment (start 89 113) (end 81 105) (width 0.2) (layer "F.Cu") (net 16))
 (segment (start 81 93) (end 80 92) (width 0.2) (layer "F.Cu") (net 16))
 (segment (start 80 92) (end 80 76) (width 0.2) (layer "F.Cu") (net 16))
 (segment (start 92 117.54) (end 92 116) (width 0.2) (layer "F.Cu") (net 16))
 (segment (start 81 105) (end 81 97) (width 0.2) (layer "F.Cu") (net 16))
 (via (at 81 97) (size 0.7) (drill 0.3) (layers "F.Cu" "B.Cu") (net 16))
 (via (at 89 113) (size 0.7) (drill 0.3) (layers "F.Cu" "B.Cu") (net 16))
 (via (at 84 75) (size 0.7) (drill 0.3) (layers "F.Cu" "B.Cu") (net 16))
 (via (at 81 93) (size 0.7) (drill 0.3) (layers "F.Cu" "B.Cu") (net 16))
 (via (at 92 116) (size 0.7) (drill 0.3) (layers "F.Cu" "B.Cu") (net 16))
 (via (at 80 76) (size 0.7) (drill 0.3) (layers "F.Cu" "B.Cu") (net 16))
 (segment (start 81 97) (end 81 93) (width 0.2) (layer "B.Cu") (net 16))
 (segment (start 81 75) (end 84 75) (width 0.2) (layer "B.Cu") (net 16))
 (segment (start 80 76) (end 81 75) (width 0.2) (layer "B.Cu") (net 16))
 (segment (start 92 116) (end 89 113) (width 0.2) (layer "B.Cu") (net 16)))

